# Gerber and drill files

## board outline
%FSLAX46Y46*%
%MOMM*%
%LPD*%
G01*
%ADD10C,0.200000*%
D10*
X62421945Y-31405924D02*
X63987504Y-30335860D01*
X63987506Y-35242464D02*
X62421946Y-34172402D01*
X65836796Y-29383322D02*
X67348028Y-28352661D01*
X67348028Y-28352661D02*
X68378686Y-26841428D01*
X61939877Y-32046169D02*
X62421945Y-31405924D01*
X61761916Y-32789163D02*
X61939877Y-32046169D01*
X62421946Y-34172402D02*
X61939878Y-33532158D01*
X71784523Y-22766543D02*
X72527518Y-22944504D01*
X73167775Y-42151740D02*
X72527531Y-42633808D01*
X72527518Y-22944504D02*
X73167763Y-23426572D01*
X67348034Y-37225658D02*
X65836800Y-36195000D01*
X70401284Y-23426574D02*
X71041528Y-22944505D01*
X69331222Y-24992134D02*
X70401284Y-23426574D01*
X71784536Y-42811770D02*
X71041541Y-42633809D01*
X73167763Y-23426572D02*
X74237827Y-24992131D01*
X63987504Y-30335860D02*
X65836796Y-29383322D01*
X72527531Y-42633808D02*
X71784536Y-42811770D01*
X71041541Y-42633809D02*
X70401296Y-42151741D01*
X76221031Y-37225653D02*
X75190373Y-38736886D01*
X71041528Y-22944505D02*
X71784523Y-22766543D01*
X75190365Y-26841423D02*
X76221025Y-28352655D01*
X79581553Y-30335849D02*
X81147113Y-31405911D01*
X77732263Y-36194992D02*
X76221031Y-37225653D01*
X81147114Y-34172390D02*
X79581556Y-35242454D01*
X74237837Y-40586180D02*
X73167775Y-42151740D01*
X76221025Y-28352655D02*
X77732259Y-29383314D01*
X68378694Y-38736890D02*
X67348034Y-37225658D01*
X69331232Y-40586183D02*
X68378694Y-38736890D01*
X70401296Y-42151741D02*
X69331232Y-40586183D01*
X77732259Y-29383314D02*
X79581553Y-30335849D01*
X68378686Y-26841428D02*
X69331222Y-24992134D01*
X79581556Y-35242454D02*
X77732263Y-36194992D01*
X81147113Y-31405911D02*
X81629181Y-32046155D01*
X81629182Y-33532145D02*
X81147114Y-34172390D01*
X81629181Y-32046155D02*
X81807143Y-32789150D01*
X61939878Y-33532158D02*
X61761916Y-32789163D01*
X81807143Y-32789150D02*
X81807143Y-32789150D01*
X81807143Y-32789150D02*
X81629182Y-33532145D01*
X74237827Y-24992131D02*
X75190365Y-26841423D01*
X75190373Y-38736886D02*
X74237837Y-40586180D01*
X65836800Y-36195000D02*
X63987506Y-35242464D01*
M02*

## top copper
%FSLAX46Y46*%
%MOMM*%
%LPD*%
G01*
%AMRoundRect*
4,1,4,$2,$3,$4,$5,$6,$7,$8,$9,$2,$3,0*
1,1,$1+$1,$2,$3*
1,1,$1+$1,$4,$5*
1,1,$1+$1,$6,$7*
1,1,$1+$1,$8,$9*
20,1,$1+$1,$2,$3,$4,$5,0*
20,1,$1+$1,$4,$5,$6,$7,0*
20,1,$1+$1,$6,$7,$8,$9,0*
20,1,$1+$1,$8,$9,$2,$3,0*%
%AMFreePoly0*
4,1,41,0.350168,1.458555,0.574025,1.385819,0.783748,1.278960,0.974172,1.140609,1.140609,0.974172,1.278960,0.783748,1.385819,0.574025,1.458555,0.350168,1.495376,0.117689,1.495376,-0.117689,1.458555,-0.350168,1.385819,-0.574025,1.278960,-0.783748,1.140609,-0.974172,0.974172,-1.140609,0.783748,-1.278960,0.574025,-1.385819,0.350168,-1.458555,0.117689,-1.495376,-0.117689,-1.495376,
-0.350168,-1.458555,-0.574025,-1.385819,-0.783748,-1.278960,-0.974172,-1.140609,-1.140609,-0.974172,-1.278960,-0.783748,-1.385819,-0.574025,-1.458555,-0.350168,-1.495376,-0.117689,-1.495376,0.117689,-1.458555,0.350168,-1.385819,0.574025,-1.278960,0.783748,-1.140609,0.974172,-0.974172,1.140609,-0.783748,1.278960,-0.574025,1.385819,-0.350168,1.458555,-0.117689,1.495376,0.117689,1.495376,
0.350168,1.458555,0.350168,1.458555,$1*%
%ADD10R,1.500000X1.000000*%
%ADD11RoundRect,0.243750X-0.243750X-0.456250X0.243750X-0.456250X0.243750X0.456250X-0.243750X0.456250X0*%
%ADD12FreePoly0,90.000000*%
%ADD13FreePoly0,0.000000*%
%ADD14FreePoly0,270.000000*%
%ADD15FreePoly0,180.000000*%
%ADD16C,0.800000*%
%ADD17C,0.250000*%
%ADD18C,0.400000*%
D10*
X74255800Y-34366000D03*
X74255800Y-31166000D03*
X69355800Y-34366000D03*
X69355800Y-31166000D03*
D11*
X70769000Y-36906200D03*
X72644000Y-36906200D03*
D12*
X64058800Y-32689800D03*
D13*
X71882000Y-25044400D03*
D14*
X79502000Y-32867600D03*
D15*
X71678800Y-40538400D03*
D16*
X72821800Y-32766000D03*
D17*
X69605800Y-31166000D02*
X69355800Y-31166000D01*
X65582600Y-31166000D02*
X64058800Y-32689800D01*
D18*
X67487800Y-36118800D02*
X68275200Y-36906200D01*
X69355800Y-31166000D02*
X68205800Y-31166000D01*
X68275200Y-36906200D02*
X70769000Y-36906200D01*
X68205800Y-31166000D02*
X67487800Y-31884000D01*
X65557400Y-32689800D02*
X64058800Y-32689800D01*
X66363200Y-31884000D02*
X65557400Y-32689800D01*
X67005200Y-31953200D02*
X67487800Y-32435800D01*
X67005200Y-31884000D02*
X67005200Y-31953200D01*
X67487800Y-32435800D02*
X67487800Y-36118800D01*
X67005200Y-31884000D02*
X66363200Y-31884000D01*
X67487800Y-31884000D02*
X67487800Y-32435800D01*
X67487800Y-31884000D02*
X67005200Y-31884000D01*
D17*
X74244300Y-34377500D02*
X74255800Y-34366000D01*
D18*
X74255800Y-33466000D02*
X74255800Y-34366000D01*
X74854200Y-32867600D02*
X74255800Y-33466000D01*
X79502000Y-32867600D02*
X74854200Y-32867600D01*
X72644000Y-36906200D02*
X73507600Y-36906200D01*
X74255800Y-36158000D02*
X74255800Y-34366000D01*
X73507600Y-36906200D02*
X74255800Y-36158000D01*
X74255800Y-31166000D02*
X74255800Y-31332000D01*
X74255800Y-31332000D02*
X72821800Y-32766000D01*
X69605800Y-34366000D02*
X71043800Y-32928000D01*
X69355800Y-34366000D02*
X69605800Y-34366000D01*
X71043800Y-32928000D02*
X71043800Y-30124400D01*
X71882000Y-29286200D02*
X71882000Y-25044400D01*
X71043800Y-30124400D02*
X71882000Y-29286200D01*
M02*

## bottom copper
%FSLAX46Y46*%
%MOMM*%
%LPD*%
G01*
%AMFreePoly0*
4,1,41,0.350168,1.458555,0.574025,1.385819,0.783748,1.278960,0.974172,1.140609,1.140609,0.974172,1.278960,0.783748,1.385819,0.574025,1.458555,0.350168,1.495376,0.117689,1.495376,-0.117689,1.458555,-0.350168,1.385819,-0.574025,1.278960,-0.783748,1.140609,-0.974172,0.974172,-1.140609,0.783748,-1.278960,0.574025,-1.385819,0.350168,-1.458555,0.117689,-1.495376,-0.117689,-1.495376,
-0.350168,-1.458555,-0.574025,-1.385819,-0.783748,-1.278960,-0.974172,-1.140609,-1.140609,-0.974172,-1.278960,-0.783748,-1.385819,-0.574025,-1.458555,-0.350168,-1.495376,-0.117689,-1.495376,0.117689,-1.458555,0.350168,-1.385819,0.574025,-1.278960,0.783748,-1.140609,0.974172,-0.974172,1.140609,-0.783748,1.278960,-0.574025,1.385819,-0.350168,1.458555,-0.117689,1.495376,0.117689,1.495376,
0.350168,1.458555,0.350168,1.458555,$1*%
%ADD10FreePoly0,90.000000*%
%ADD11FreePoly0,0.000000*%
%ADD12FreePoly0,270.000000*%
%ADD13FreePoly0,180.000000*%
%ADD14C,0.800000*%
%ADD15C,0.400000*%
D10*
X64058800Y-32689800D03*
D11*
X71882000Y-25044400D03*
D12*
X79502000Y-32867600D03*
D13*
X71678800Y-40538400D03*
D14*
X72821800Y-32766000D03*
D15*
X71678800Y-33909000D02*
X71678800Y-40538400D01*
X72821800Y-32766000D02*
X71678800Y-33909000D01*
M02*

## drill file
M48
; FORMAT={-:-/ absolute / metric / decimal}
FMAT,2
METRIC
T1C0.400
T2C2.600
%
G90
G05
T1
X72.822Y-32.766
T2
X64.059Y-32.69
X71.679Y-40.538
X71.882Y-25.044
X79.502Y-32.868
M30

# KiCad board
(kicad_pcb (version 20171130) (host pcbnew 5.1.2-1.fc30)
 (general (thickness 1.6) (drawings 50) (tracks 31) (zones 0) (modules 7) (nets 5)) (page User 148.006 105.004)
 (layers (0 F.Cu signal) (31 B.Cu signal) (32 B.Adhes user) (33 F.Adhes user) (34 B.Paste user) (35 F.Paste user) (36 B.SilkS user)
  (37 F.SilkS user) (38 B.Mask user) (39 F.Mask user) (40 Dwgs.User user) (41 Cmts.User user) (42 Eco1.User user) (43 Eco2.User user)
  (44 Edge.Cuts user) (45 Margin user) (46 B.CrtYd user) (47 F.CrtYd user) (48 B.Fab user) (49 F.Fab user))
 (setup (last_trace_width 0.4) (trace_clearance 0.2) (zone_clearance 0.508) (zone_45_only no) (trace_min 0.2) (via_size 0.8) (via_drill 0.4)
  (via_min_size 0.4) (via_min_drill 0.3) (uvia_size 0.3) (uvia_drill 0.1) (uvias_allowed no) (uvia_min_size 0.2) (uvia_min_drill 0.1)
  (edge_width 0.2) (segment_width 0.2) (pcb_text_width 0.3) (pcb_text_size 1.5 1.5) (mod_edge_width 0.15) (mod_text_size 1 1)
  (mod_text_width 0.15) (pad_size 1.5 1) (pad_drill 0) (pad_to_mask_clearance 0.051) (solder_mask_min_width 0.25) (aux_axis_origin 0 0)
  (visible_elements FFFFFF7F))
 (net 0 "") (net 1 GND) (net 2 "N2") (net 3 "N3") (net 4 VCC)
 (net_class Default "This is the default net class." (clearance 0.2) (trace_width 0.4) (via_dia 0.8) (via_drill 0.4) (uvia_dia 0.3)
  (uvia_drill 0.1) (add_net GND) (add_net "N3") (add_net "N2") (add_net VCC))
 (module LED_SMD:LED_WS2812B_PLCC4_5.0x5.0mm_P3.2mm (layer F.Cu) (at 71.8058 32.766)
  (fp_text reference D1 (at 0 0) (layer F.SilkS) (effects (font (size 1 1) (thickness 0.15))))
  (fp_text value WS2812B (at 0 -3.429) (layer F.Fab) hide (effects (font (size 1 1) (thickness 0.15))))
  (pad 3 smd rect (at 2.45 1.6) (size 1.5 1) (layers F.Cu F.Paste F.Mask) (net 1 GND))
  (pad 4 smd rect (at 2.45 -1.6) (size 1.5 1) (layers F.Cu F.Paste F.Mask) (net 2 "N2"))
  (pad 2 smd rect (at -2.45 1.6) (size 1.5 1) (layers F.Cu F.Paste F.Mask) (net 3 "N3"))
  (pad 1 smd rect (at -2.45 -1.6) (size 1.5 1) (layers F.Cu F.Paste F.Mask) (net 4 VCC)))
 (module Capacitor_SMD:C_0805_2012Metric (layer F.Cu) (at 71.7065 36.9062)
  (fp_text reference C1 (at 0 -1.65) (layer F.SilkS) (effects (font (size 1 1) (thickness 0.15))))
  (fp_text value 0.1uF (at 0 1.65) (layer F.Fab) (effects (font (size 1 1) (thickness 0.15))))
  (pad 1 smd roundrect (at -0.9375 0) (size 0.975 1.4) (layers F.Cu F.Paste F.Mask) (roundrect_rratio 0.25) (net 4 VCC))
  (pad 2 smd roundrect (at 0.9375 0) (size 0.975 1.4) (layers F.Cu F.Paste F.Mask) (roundrect_rratio 0.25) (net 1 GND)))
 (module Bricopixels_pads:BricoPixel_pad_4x (layer F.Cu) (at 64.0588 32.6898 90)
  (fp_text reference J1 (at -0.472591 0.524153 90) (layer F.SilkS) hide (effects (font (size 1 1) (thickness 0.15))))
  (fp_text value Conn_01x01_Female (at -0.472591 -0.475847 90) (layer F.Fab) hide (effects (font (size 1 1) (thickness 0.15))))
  (pad 1 thru_hole custom (at 0 0 90) (size 3 3) (drill 2.6) (layers *.Cu *.Mask) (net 4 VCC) (zone_connect 0)
   (options (clearance outline) (anchor circle)) (primitives)))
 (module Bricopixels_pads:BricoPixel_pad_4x (layer F.Cu) (at 71.882 25.0444)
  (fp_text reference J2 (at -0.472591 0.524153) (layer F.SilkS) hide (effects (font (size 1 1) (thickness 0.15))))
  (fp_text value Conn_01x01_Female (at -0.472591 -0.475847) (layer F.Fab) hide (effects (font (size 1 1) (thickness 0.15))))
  (pad 1 thru_hole custom (at 0 0) (size 3 3) (drill 2.6) (layers *.Cu *.Mask) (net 3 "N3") (zone_connect 0)
   (options (clearance outline) (anchor circle)) (primitives)))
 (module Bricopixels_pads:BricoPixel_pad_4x (layer F.Cu) (at 79.502 32.8676 270)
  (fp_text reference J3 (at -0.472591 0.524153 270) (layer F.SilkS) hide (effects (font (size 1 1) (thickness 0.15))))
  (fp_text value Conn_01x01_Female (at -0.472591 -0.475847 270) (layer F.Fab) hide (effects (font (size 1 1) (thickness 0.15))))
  (pad 1 thru_hole custom (at 0 0 270) (size 3 3) (drill 2.6) (layers *.Cu *.Mask) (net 1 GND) (zone_connect 0)
   (options (clearance outline) (anchor circle)) (primitives)))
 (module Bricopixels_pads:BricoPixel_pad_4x (layer F.Cu) (at 71.6788 40.5384 180)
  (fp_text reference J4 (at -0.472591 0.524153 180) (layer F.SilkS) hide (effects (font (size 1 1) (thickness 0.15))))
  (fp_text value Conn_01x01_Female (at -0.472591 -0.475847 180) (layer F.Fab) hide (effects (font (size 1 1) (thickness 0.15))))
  (pad 1 thru_hole custom (at 0 0 180) (size 3 3) (drill 2.6) (layers *.Cu *.Mask) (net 2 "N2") (zone_connect 0)
   (options (clearance outline) (anchor circle)) (primitives)))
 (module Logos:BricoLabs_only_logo (layer B.Cu) (at 71.882 32.0548 180)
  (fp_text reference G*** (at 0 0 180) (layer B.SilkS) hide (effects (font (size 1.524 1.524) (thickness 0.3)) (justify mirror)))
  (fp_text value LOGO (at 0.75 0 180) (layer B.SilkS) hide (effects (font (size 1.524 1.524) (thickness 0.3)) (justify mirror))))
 (gr_line (start 62.421945 31.405924) (end 63.987504 30.33586) (layer Edge.Cuts) (width 0.2))
 (gr_line (start 63.987506 35.242464) (end 62.421946 34.172402) (layer Edge.Cuts) (width 0.2))
 (gr_line (start 65.836796 29.383322) (end 67.348028 28.352661) (layer Edge.Cuts) (width 0.2))
 (gr_line (start 67.348028 28.352661) (end 68.378686 26.841428) (layer Edge.Cuts) (width 0.2))
 (gr_line (start 61.939877 32.046169) (end 62.421945 31.405924) (layer Edge.Cuts) (width 0.2))
 (gr_line (start 61.761916 32.789163) (end 61.939877 32.046169) (layer Edge.Cuts) (width 0.2))
 (gr_line (start 62.421946 34.172402) (end 61.939878 33.532158) (layer Edge.Cuts) (width 0.2))
 (gr_line (start 71.784523 22.766543) (end 72.527518 22.944504) (layer Edge.Cuts) (width 0.2))
 (gr_line (start 73.167775 42.15174) (end 72.527531 42.633808) (layer Edge.Cuts) (width 0.2))
 (gr_line (start 72.527518 22.944504) (end 73.167763 23.426572) (layer Edge.Cuts) (width 0.2))
 (gr_line (start 67.348034 37.225658) (end 65.8368 36.195) (layer Edge.Cuts) (width 0.2))
 (gr_line (start 70.401284 23.426574) (end 71.041528 22.944505) (layer Edge.Cuts) (width 0.2))
 (gr_line (start 69.331222 24.992134) (end 70.401284 23.426574) (layer Edge.Cuts) (width 0.2))
 (gr_line (start 71.784536 42.81177) (end 71.041541 42.633809) (layer Edge.Cuts) (width 0.2))
 (gr_line (start 73.167763 23.426572) (end 74.237827 24.992131) (layer Edge.Cuts) (width 0.2))
 (gr_line (start 63.987504 30.33586) (end 65.836796 29.383322) (layer Edge.Cuts) (width 0.2))
 (gr_line (start 72.527531 42.633808) (end 71.784536 42.81177) (layer Edge.Cuts) (width 0.2))
 (gr_line (start 71.041541 42.633809) (end 70.401296 42.151741) (layer Edge.Cuts) (width 0.2))
 (gr_line (start 76.221031 37.225653) (end 75.190373 38.736886) (layer Edge.Cuts) (width 0.2))
 (gr_line (start 71.041528 22.944505) (end 71.784523 22.766543) (layer Edge.Cuts) (width 0.2))
 (gr_line (start 75.190365 26.841423) (end 76.221025 28.352655) (layer Edge.Cuts) (width 0.2))
 (gr_line (start 79.581553 30.335849) (end 81.147113 31.405911) (layer Edge.Cuts) (width 0.2))
 (gr_line (start 77.732263 36.194992) (end 76.221031 37.225653) (layer Edge.Cuts) (width 0.2))
 (gr_line (start 81.147114 34.17239) (end 79.581556 35.242454) (layer Edge.Cuts) (width 0.2))
 (gr_line (start 74.237837 40.58618) (end 73.167775 42.15174) (layer Edge.Cuts) (width 0.2))
 (gr_line (start 76.221025 28.352655) (end 77.732259 29.383314) (layer Edge.Cuts) (width 0.2))
 (gr_line (start 68.378694 38.73689) (end 67.348034 37.225658) (layer Edge.Cuts) (width 0.2))
 (gr_line (start 69.331232 40.586183) (end 68.378694 38.73689) (layer Edge.Cuts) (width 0.2))
 (gr_line (start 70.401296 42.151741) (end 69.331232 40.586183) (layer Edge.Cuts) (width 0.2))
 (gr_line (start 77.732259 29.383314) (end 79.581553 30.335849) (layer Edge.Cuts) (width 0.2))
 (gr_line (start 68.378686 26.841428) (end 69.331222 24.992134) (layer Edge.Cuts) (width 0.2))
 (gr_line (start 79.581556 35.242454) (end 77.732263 36.194992) (layer Edge.Cuts) (width 0.2))
 (gr_line (start 81.147113 31.405911) (end 81.629181 32.046155) (layer Edge.Cuts) (width 0.2))
 (gr_line (start 81.629182 33.532145) (end 81.147114 34.17239) (layer Edge.Cuts) (width 0.2))
 (gr_line (start 81.629181 32.046155) (end 81.807143 32.78915) (layer Edge.Cuts) (width 0.2))
 (gr_line (start 61.939878 33.532158) (end 61.761916 32.789163) (layer Edge.Cuts) (width 0.2))
 (gr_line (start 81.807143 32.78915) (end 81.807143 32.78915) (layer Edge.Cuts) (width 0.2))
 (gr_line (start 81.807143 32.78915) (end 81.629182 33.532145) (layer Edge.Cuts) (width 0.2))
 (gr_line (start 74.237827 24.992131) (end 75.190365 26.841423) (layer Edge.Cuts) (width 0.2))
 (gr_line (start 75.190373 38.736886) (end 74.237837 40.58618) (layer Edge.Cuts) (width 0.2))
 (gr_line (start 65.8368 36.195) (end 63.987506 35.242464) (layer Edge.Cuts) (width 0.2))
 (segment (start 69.6058 31.166) (end 69.3558 31.166) (width 0.25) (layer F.Cu) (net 4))
 (segment (start 65.5826 31.166) (end 64.0588 32.6898) (width 0.25) (layer F.Cu) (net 4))
 (segment (start 67.4878 36.1188) (end 68.2752 36.9062) (width 0.4) (layer F.Cu) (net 4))
 (segment (start 69.3558 31.166) (end 68.2058 31.166) (width 0.4) (layer F.Cu) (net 4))
 (segment (start 68.2752 36.9062) (end 70.769 36.9062) (width 0.4) (layer F.Cu) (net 4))
 (segment (start 68.2058 31.166) (end 67.4878 31.884) (width 0.4) (layer F.Cu) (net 4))
 (segment (start 65.5574 32.6898) (end 64.0588 32.6898) (width 0.4) (layer F.Cu) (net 4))
 (segment (start 66.3632 31.884) (end 65.5574 32.6898) (width 0.4) (layer F.Cu) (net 4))
 (segment (start 67.0052 31.9532) (end 67.4878 32.4358) (width 0.4) (layer F.Cu) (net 4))
 (segment (start 67.0052 31.884) (end 67.0052 31.9532) (width 0.4) (layer F.Cu) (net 4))
 (segment (start 67.4878 32.4358) (end 67.4878 36.1188) (width 0.4) (layer F.Cu) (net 4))
 (segment (start 67.0052 31.884) (end 66.3632 31.884) (width 0.4) (layer F.Cu) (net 4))
 (segment (start 67.4878 31.884) (end 67.4878 32.4358) (width 0.4) (layer F.Cu) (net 4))
 (segment (start 67.4878 31.884) (end 67.0052 31.884) (width 0.4) (layer F.Cu) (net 4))
 (segment (start 74.2443 34.3775) (end 74.2558 34.366) (width 0.25) (layer F.Cu) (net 1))
 (segment (start 74.2558 33.466) (end 74.2558 34.366) (width 0.4) (layer F.Cu) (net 1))
 (segment (start 74.8542 32.8676) (end 74.2558 33.466) (width 0.4) (layer F.Cu) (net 1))
 (segment (start 79.502 32.8676) (end 74.8542 32.8676) (width 0.4) (layer F.Cu) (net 1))
 (segment (start 72.644 36.9062) (end 73.5076 36.9062) (width 0.4) (layer F.Cu) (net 1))
 (segment (start 74.2558 36.158) (end 74.2558 34.366) (width 0.4) (layer F.Cu) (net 1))
 (segment (start 73.5076 36.9062) (end 74.2558 36.158) (width 0.4) (layer F.Cu) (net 1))
 (via (at 72.8218 32.766) (size 0.8) (drill 0.4) (layers F.Cu B.Cu) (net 2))
 (segment (start 74.2558 31.166) (end 74.2558 31.332) (width 0.4) (layer F.Cu) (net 2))
 (segment (start 74.2558 31.332) (end 72.8218 32.766) (width 0.4) (layer F.Cu) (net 2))
 (segment (start 71.6788 33.909) (end 71.6788 40.5384) (width 0.4) (layer B.Cu) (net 2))
 (segment (start 72.8218 32.766) (end 71.6788 33.909) (width 0.4) (layer B.Cu) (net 2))
 (segment (start 69.6058 34.366) (end 71.0438 32.928) (width 0.4) (layer F.Cu) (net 3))
 (segment (start 69.3558 34.366) (end 69.6058 34.366) (width 0.4) (layer F.Cu) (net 3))
 (segment (start 71.0438 32.928) (end 71.0438 30.1244) (width 0.4) (layer F.Cu) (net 3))
 (segment (start 71.882 29.2862) (end 71.882 25.0444) (width 0.4) (layer F.Cu) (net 3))
 (segment (start 71.0438 30.1244) (end 71.882 29.2862) (width 0.4) (layer F.Cu) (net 3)))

